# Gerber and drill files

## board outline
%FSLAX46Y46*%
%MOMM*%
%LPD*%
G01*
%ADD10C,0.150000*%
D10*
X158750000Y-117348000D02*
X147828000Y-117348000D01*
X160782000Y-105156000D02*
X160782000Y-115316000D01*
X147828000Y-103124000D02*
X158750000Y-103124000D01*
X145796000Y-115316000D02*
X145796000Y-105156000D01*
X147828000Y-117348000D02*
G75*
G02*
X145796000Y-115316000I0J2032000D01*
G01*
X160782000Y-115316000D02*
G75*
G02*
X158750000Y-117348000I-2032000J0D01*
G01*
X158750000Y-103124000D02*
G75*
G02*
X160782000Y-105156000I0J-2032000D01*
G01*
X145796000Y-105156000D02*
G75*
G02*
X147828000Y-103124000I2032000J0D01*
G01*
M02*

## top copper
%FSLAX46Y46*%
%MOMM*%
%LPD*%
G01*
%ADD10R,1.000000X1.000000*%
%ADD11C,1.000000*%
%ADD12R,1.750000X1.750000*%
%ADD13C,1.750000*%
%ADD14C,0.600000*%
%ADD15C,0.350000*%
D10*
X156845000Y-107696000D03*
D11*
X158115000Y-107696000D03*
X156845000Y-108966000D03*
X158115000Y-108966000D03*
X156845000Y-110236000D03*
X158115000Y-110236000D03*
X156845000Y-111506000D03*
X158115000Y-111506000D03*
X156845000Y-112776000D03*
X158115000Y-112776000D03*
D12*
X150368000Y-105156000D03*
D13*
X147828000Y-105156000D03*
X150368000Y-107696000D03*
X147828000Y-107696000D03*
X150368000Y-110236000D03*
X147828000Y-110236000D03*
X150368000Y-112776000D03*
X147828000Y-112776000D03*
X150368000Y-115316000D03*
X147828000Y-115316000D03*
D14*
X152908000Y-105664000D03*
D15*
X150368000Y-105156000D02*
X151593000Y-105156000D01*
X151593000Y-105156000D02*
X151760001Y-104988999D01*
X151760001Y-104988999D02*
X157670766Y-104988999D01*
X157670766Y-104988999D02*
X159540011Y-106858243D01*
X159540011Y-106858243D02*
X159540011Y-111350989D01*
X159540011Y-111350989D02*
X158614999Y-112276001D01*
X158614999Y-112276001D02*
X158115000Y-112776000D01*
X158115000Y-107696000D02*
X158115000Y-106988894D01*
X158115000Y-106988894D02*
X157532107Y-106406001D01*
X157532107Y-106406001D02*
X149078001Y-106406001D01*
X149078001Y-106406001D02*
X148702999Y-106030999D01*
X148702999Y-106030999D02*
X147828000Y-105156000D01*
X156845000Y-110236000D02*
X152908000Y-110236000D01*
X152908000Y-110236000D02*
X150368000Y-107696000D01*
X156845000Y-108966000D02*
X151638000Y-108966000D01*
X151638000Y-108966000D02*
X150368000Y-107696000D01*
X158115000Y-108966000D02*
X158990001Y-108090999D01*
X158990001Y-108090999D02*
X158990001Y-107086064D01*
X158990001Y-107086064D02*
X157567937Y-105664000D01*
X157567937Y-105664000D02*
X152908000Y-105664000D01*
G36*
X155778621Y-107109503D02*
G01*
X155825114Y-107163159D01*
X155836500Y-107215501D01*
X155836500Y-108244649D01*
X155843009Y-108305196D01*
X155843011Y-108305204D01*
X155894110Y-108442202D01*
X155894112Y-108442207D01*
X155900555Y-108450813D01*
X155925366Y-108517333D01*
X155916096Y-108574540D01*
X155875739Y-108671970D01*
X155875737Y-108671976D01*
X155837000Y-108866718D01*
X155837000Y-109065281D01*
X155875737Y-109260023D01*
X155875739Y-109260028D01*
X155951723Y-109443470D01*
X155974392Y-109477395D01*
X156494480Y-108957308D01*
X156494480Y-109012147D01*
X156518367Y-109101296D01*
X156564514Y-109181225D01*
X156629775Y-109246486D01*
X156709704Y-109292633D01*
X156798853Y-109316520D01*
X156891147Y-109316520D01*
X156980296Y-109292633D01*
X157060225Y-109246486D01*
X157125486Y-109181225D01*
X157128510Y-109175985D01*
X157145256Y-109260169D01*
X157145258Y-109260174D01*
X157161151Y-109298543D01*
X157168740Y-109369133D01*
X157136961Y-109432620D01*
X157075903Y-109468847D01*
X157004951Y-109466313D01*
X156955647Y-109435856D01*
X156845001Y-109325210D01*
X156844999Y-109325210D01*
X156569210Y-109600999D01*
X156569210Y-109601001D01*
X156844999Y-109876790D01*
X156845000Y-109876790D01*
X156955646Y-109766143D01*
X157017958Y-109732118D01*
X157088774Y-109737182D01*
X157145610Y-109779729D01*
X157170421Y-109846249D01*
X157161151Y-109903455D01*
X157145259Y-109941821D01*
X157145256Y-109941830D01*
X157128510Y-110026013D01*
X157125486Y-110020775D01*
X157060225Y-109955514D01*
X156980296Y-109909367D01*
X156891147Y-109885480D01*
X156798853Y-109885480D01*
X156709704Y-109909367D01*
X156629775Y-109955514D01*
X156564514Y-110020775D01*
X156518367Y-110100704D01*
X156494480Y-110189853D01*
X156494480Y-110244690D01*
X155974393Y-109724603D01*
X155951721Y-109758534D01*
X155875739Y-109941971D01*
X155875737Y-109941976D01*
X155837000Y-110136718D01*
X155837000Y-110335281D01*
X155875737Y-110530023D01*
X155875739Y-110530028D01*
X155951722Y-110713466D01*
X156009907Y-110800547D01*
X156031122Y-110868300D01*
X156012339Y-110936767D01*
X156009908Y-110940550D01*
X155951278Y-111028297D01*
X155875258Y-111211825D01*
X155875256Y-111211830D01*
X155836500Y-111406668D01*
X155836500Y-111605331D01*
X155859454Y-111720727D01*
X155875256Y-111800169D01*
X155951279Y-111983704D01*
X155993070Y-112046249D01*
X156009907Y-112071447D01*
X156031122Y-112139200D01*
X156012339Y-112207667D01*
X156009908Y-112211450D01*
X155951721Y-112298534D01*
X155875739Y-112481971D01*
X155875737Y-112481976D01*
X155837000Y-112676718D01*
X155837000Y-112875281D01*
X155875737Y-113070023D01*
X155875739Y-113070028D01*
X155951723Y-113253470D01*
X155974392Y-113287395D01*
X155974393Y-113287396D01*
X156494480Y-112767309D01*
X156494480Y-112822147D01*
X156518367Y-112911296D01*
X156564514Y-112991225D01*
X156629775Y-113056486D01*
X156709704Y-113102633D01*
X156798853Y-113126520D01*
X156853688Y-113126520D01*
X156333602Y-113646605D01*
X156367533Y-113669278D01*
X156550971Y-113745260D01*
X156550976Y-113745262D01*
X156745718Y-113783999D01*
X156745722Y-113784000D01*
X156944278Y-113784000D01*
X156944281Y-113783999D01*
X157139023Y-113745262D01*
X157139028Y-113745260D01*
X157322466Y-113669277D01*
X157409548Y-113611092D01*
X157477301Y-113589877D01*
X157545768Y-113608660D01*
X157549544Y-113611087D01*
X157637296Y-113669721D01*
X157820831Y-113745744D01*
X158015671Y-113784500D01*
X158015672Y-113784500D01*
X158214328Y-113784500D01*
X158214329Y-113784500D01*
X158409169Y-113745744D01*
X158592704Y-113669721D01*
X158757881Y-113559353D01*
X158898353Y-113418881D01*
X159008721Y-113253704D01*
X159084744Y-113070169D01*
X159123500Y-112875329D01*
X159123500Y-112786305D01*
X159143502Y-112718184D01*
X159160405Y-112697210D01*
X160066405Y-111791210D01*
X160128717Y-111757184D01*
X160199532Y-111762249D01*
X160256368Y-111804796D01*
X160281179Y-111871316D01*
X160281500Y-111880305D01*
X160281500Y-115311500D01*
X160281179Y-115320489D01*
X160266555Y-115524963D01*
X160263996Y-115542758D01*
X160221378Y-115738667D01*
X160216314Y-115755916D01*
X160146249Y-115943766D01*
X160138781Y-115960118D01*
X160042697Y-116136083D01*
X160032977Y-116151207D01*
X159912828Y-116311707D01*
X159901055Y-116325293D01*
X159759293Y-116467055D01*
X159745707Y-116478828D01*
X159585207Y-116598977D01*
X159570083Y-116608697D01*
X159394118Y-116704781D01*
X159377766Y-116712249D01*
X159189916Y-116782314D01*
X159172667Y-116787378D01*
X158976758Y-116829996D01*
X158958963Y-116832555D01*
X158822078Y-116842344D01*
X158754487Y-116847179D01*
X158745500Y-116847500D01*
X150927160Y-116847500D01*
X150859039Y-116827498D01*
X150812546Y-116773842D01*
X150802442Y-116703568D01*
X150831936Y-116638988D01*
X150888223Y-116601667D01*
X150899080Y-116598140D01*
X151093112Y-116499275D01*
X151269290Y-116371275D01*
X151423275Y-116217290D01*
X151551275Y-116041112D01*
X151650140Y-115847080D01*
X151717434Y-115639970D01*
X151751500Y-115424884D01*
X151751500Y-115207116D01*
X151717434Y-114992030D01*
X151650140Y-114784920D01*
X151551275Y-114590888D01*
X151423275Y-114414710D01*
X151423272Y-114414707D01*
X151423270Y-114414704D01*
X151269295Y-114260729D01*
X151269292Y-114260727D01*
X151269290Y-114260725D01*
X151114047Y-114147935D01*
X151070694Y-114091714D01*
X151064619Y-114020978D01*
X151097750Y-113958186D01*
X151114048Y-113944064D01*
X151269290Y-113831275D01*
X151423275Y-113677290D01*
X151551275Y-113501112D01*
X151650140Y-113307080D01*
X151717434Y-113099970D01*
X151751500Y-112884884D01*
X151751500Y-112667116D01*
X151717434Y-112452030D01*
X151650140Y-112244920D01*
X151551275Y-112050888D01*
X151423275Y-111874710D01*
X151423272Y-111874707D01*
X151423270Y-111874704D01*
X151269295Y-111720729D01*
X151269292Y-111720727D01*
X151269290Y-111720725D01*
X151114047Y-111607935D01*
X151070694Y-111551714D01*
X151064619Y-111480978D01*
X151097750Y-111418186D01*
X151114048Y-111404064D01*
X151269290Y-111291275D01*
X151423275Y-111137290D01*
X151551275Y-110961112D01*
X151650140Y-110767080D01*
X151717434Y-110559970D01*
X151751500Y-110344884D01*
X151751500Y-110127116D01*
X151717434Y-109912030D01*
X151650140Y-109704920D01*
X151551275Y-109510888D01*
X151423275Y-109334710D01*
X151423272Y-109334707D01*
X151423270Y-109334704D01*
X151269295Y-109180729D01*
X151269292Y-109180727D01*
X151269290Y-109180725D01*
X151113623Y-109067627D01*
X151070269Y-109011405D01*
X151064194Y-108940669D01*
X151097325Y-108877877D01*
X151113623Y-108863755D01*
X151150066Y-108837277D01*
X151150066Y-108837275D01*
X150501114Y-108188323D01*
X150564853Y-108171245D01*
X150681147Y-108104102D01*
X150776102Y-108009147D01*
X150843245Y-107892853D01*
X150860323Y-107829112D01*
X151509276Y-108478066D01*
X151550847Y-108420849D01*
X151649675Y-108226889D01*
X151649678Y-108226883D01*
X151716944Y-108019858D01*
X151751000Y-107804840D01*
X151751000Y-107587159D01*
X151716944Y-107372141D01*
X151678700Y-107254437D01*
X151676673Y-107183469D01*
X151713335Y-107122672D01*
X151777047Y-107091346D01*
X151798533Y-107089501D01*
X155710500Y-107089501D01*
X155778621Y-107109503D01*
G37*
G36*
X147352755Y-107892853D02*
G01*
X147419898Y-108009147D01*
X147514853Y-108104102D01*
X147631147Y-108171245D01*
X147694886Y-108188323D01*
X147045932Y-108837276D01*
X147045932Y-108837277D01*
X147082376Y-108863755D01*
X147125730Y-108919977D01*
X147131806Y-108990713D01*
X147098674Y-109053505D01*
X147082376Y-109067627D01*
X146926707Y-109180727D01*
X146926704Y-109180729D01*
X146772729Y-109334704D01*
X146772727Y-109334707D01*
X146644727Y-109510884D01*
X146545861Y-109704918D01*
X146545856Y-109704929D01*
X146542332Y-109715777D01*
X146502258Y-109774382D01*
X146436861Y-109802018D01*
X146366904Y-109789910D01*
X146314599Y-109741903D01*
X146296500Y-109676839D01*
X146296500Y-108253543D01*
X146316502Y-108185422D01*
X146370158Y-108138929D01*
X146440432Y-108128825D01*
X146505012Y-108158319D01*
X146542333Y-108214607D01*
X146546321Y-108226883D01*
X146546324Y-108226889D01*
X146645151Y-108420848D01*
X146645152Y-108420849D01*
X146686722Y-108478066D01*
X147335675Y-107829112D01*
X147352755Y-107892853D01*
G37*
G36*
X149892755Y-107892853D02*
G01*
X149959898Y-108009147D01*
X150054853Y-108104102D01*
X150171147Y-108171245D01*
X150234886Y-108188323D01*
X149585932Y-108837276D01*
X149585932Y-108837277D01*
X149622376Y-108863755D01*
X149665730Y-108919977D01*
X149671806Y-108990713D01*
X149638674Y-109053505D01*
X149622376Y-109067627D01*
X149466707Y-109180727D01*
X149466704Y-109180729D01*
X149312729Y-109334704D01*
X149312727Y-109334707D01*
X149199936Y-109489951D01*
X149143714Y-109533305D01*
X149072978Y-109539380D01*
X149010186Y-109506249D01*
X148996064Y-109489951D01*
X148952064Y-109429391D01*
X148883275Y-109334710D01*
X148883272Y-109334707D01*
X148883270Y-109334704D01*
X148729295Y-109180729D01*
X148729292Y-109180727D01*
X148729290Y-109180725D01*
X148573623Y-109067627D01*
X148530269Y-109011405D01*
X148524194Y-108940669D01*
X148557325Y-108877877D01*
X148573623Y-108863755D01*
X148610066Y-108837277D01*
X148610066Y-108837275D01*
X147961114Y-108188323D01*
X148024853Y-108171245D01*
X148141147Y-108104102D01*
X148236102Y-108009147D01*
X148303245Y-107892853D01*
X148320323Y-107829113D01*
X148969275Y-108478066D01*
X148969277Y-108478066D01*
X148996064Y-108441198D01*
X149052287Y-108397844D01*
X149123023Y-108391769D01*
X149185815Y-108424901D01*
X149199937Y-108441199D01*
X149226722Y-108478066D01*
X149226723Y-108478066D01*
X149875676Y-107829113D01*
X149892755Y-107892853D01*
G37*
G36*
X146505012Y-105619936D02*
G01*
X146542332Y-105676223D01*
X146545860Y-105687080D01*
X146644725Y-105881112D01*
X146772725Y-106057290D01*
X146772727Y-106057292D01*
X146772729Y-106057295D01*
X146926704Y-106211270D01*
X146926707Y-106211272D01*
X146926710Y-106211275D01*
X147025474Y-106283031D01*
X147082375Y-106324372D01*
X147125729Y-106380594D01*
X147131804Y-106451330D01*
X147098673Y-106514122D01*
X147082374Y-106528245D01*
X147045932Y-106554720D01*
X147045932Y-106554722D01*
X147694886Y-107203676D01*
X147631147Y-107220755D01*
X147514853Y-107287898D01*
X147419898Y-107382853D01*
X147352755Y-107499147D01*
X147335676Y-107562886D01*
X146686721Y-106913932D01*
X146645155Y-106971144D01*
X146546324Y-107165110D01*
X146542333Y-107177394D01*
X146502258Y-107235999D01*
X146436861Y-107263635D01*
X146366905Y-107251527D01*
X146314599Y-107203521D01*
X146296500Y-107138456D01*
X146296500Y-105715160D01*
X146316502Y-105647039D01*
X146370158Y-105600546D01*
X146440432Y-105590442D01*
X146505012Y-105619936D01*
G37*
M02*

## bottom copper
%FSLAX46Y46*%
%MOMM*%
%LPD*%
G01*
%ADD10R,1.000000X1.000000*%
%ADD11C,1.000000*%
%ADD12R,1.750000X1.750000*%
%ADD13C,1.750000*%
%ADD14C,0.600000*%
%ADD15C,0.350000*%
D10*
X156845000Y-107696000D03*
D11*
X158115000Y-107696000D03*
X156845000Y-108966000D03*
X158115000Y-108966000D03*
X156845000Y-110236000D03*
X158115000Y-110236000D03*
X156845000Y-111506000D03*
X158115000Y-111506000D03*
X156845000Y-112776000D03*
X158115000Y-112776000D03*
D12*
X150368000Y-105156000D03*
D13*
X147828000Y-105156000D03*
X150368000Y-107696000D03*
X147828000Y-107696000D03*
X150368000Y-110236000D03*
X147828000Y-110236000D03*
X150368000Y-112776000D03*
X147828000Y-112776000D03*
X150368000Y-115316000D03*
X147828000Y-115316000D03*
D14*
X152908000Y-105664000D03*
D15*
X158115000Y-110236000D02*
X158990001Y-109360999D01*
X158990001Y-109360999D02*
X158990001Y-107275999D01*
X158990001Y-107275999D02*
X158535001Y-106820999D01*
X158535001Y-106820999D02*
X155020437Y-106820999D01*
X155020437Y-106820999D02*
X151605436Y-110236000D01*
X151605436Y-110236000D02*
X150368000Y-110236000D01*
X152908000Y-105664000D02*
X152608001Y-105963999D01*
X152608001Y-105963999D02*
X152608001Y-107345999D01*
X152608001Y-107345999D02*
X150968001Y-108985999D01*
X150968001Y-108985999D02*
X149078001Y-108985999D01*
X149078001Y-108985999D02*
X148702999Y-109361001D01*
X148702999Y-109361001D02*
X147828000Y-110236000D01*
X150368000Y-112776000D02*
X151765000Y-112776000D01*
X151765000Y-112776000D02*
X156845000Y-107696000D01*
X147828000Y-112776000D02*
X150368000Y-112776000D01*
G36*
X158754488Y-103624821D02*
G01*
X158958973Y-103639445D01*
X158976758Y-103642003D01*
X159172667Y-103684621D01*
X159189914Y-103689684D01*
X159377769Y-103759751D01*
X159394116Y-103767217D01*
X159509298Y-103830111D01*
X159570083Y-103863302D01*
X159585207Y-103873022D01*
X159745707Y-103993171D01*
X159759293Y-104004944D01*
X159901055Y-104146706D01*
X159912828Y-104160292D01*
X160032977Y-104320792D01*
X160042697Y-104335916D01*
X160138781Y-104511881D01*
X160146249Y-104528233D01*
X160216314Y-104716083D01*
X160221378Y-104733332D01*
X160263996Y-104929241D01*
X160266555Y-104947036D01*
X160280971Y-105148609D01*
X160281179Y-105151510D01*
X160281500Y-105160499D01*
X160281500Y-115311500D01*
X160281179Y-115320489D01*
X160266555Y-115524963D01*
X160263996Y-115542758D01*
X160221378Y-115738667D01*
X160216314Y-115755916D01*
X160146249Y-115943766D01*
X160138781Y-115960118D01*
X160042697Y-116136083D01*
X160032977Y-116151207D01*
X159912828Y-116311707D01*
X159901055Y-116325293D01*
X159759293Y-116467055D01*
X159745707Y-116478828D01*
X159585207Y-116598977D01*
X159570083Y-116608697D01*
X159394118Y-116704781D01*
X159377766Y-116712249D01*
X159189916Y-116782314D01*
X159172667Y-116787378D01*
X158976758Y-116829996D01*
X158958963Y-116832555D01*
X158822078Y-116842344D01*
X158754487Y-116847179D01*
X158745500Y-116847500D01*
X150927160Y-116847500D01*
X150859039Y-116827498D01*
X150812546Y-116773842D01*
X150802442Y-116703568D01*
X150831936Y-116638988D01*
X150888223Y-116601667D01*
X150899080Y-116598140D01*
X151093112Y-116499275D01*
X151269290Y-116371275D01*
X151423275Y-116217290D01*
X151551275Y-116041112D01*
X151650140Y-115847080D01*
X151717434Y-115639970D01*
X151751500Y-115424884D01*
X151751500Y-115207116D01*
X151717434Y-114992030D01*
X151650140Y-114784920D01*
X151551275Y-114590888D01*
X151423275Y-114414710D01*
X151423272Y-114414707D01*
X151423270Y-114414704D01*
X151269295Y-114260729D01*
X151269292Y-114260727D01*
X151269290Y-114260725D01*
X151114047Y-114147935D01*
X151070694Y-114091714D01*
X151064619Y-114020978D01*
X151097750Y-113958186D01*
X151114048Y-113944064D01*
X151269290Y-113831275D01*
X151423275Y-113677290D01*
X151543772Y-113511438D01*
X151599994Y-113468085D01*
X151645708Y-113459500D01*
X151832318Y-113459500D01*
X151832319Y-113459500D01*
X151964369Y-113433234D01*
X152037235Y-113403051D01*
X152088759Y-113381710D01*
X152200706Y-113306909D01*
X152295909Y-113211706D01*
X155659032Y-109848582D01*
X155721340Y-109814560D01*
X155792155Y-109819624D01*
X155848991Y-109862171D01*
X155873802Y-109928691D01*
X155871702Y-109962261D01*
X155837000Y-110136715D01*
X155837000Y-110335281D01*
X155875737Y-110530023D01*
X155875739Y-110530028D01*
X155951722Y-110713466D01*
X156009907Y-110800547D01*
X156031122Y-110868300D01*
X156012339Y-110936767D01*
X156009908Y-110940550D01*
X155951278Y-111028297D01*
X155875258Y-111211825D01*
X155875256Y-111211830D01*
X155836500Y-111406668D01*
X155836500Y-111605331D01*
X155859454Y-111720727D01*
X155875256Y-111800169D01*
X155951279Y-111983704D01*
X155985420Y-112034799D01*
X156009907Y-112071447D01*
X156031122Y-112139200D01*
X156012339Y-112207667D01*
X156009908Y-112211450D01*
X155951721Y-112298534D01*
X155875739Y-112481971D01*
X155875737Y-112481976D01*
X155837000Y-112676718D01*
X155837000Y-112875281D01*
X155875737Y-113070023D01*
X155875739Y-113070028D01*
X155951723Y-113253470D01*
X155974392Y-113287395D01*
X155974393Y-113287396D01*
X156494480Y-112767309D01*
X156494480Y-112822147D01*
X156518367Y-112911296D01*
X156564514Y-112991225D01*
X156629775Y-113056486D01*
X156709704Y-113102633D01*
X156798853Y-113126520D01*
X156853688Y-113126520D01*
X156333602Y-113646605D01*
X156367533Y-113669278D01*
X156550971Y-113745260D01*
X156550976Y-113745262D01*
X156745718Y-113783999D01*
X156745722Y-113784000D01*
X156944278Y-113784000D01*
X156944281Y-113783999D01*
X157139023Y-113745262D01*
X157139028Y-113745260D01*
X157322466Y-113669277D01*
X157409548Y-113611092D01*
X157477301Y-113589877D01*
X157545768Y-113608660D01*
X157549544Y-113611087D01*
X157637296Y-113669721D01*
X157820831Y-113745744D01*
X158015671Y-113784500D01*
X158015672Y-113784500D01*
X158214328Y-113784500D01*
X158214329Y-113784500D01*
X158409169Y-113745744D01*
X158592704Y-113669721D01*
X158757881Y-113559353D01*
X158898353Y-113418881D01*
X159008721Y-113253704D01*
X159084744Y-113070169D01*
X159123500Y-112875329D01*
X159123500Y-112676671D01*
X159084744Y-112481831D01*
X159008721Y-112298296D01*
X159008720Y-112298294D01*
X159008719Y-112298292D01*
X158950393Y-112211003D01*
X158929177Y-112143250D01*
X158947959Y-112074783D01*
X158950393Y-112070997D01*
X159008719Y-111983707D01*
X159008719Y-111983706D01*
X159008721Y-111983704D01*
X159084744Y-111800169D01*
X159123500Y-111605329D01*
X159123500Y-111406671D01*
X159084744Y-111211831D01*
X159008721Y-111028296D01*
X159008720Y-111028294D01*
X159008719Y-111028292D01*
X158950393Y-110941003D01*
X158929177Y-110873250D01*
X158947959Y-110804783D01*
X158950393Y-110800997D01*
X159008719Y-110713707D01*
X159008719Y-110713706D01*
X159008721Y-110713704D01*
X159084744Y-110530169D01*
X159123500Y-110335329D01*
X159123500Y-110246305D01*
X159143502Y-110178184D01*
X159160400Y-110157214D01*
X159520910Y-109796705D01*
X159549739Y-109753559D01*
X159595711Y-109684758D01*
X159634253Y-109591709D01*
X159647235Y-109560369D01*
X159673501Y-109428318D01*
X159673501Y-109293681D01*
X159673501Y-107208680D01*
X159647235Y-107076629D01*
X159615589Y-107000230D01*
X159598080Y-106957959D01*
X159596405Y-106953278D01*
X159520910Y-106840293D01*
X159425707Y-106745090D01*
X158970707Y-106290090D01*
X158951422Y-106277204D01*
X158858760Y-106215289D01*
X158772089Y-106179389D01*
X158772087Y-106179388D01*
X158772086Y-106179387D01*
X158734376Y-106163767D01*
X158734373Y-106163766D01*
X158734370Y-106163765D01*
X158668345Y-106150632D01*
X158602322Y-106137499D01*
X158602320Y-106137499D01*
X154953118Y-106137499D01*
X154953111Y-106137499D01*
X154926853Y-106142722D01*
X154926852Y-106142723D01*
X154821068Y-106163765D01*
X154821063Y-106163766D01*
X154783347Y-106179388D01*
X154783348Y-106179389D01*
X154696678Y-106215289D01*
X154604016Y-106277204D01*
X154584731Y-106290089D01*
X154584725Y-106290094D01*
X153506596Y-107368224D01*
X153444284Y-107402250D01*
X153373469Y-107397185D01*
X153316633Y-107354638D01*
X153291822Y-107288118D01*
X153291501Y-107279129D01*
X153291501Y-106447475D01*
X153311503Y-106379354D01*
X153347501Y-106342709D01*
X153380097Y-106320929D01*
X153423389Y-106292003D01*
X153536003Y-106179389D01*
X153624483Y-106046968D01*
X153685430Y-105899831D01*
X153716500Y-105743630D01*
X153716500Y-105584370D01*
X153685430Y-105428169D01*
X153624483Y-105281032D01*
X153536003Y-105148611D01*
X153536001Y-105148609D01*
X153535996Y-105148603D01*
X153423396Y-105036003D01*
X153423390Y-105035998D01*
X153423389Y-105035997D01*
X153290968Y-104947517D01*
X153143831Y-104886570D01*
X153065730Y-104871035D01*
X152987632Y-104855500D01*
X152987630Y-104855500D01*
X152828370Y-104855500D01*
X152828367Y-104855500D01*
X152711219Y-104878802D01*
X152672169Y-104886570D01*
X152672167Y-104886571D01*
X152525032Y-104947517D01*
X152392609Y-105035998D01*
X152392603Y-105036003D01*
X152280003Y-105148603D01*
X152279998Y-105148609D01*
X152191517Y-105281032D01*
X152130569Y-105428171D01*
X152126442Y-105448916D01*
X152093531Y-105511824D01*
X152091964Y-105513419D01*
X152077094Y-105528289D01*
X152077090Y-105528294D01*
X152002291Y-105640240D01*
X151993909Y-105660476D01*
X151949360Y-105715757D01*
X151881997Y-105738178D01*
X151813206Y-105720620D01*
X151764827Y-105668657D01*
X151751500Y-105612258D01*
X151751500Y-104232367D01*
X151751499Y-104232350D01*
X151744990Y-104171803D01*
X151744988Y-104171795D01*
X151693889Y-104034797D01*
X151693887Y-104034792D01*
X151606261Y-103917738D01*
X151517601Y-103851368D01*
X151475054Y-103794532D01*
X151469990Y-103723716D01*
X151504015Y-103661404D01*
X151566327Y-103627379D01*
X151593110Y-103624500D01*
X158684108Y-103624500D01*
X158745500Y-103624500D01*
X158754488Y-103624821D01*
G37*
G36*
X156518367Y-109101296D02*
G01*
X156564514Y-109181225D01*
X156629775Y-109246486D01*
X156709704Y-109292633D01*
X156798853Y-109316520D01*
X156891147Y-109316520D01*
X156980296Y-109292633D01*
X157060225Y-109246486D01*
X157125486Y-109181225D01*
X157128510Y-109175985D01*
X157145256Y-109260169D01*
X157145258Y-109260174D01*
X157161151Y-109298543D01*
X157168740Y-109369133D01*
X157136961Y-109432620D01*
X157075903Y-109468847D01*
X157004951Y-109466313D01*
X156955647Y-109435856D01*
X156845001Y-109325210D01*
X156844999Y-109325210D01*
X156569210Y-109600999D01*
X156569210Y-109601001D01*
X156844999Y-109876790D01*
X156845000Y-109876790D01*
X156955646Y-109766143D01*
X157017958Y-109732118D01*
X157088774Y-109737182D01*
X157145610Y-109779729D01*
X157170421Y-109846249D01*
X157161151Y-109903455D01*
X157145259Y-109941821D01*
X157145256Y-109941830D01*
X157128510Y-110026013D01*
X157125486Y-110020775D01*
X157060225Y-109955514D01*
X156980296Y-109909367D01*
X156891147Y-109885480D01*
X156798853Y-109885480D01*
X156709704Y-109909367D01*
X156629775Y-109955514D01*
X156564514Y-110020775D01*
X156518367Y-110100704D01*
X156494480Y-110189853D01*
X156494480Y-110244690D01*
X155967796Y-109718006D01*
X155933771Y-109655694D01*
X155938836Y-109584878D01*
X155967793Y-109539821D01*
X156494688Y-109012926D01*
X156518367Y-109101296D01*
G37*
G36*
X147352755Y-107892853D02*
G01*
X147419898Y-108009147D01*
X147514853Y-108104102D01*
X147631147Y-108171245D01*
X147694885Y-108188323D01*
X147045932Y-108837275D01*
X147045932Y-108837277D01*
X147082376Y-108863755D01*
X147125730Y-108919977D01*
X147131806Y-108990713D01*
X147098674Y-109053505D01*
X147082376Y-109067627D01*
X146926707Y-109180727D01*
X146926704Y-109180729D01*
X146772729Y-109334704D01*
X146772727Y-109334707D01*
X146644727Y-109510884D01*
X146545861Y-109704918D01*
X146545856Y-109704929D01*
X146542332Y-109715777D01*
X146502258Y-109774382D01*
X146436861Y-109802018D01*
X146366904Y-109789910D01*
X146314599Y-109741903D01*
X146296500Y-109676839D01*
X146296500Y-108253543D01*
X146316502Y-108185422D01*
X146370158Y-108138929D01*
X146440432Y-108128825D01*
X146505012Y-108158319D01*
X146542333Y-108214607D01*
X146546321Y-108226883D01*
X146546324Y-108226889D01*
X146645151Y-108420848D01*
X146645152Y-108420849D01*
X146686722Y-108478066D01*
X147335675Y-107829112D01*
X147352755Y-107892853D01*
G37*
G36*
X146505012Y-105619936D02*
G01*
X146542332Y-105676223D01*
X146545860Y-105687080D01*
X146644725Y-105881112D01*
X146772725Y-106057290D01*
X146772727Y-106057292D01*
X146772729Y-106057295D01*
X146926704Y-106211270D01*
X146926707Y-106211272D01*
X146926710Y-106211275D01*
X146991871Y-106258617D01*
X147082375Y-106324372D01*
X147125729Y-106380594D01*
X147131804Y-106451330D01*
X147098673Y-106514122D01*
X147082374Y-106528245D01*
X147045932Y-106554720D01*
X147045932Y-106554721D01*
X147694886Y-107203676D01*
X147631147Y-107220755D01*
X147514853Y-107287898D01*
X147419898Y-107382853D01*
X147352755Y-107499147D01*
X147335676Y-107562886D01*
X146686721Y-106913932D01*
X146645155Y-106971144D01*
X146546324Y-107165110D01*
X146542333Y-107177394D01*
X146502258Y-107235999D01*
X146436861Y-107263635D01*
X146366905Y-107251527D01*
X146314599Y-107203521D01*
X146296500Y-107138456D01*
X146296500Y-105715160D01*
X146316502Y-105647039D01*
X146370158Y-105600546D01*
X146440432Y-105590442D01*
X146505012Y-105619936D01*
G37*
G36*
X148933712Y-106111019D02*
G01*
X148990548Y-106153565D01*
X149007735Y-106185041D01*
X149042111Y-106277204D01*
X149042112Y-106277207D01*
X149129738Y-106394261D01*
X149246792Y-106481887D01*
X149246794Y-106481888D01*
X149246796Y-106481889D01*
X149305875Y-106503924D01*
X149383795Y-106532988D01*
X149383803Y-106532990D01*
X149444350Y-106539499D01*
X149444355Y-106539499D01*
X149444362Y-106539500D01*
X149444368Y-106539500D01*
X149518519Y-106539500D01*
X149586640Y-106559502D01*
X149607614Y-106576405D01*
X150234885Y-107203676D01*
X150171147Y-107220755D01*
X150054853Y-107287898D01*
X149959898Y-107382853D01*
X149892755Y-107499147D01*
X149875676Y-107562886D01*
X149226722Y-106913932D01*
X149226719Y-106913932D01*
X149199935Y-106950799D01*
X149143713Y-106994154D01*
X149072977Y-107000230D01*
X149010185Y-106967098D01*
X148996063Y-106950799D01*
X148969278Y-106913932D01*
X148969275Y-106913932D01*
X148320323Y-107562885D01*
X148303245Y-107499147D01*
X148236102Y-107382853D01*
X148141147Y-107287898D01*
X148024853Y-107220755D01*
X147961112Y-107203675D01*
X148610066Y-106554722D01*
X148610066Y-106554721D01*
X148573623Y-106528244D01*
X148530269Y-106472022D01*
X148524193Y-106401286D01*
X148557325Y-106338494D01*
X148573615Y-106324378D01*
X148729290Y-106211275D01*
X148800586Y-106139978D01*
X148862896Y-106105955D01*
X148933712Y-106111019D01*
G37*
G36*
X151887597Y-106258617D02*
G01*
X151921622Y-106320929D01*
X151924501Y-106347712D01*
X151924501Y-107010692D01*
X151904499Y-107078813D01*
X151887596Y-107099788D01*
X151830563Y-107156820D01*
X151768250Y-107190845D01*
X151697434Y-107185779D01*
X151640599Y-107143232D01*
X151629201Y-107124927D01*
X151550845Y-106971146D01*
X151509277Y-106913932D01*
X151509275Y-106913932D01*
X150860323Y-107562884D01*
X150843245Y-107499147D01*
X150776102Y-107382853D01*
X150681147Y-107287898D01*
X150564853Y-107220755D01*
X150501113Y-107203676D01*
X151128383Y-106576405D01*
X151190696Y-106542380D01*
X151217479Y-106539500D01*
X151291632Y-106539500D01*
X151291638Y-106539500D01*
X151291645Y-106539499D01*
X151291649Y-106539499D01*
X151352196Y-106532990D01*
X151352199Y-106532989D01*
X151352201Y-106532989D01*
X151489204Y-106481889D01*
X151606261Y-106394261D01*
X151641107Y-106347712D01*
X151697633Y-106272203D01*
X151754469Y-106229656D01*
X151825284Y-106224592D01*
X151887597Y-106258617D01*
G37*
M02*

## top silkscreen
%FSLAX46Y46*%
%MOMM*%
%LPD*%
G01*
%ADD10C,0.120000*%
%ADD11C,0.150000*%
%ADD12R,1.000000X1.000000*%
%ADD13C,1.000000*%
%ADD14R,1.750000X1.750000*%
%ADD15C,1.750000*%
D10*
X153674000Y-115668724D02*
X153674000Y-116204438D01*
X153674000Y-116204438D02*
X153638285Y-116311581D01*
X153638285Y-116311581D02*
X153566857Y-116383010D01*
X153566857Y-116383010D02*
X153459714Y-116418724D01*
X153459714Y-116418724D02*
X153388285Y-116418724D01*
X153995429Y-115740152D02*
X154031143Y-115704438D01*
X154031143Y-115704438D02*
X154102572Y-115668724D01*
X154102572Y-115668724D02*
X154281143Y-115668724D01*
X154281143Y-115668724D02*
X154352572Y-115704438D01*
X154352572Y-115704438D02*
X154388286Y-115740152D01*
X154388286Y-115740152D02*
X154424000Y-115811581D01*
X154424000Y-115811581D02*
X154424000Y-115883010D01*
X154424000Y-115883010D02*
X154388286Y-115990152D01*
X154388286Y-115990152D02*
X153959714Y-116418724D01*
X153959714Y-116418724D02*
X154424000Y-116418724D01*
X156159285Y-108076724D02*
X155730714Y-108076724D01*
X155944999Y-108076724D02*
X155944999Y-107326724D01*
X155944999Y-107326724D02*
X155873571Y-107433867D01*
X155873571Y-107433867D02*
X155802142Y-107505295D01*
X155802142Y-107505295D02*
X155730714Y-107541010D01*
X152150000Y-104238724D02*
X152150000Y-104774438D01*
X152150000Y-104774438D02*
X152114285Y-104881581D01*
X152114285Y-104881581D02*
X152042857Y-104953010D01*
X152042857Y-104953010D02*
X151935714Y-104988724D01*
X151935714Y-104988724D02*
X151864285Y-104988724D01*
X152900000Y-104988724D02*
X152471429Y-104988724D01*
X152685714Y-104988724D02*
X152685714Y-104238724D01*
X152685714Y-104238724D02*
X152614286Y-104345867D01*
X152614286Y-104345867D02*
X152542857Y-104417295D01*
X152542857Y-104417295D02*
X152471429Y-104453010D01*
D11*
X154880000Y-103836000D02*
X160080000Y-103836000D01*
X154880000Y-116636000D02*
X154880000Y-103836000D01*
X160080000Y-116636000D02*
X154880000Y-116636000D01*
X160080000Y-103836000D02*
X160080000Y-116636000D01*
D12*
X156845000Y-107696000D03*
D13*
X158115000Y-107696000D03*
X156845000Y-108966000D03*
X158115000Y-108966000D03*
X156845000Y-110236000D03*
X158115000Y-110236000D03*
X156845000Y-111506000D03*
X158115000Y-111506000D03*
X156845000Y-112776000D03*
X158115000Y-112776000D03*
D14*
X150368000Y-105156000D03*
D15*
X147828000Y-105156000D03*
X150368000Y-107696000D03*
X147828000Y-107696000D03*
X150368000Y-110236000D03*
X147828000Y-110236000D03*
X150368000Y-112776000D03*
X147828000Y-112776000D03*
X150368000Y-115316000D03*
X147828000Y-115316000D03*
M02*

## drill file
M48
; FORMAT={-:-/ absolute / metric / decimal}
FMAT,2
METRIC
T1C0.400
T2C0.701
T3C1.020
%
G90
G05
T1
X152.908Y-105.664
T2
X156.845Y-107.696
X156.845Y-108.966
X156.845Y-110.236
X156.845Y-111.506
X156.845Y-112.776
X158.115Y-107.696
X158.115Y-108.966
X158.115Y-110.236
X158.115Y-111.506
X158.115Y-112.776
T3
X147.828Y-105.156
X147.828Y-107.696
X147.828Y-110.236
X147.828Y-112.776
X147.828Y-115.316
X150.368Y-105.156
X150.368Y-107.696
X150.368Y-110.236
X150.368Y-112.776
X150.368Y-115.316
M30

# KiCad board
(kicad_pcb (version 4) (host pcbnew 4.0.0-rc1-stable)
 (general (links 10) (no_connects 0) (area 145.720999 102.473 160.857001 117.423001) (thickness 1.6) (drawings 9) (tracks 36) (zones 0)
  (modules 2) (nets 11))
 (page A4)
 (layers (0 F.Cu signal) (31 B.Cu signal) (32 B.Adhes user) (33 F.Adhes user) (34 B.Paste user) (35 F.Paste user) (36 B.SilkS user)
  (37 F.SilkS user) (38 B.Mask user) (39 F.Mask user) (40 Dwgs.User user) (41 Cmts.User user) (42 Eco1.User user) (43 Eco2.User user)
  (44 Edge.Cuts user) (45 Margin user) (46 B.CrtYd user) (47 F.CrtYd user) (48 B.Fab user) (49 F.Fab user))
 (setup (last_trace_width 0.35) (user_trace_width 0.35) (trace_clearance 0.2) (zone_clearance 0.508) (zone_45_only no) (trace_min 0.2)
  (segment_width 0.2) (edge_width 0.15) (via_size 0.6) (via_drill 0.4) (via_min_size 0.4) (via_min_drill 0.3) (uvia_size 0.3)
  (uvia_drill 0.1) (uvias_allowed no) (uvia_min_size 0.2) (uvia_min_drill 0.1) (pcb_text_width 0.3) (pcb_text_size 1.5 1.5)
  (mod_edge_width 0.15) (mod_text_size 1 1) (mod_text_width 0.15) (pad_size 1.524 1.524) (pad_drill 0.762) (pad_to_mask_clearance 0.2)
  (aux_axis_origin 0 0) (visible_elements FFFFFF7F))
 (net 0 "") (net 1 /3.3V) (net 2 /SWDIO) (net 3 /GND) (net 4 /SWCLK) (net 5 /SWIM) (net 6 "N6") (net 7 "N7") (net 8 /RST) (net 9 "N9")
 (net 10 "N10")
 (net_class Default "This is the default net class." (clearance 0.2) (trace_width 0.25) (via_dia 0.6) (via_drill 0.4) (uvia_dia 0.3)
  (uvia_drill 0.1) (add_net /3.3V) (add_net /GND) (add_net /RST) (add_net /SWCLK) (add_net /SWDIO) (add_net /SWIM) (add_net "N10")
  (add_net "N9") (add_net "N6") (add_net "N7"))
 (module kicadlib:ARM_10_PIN (layer F.Cu) (at 157.48 110.236)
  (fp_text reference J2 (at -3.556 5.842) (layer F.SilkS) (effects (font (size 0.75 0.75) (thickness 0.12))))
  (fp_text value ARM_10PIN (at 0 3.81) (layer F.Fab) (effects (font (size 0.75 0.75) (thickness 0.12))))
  (fp_line (start -2.6 -6.4) (end 2.6 -6.4) (layer F.SilkS) (width 0.15))
  (fp_line (start -2.6 6.4) (end -2.6 -6.4) (layer F.SilkS) (width 0.15))
  (fp_line (start 2.6 6.4) (end -2.6 6.4) (layer F.SilkS) (width 0.15))
  (fp_line (start 2.6 -6.4) (end 2.6 6.4) (layer F.SilkS) (width 0.15))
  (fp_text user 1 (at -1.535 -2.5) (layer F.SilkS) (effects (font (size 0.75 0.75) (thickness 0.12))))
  (pad 1 thru_hole rect (at -0.635 -2.54) (size 1 1) (drill 0.70104) (layers *.Cu *.Mask F.SilkS) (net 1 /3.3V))
  (pad 2 thru_hole circle (at 0.635 -2.54) (size 1 1) (drill 0.70104) (layers *.Cu *.Mask F.SilkS) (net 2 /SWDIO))
  (pad 3 thru_hole circle (at -0.635 -1.27) (size 1 1) (drill 0.70104) (layers *.Cu *.Mask F.SilkS) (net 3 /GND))
  (pad 4 thru_hole circle (at 0.635 -1.27) (size 1 1) (drill 0.70104) (layers *.Cu *.Mask F.SilkS) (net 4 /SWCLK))
  (pad 5 thru_hole circle (at -0.635 0) (size 1 1) (drill 0.70104) (layers *.Cu *.Mask F.SilkS) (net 3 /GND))
  (pad 6 thru_hole circle (at 0.635 0) (size 1 1) (drill 0.70104) (layers *.Cu *.Mask F.SilkS) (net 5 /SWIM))
  (pad 7 thru_hole circle (at -0.635 1.27) (size 1 1) (drill 0.70104) (layers *.Cu *.Mask F.SilkS) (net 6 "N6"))
  (pad 8 thru_hole circle (at 0.635 1.27) (size 1 1) (drill 0.70104) (layers *.Cu *.Mask F.SilkS) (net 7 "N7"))
  (pad 9 thru_hole circle (at -0.635 2.54) (size 1 1) (drill 0.70104) (layers *.Cu *.Mask F.SilkS) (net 3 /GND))
  (pad 10 thru_hole circle (at 0.635 2.54) (size 1 1) (drill 0.70104) (layers *.Cu *.Mask F.SilkS) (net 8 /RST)))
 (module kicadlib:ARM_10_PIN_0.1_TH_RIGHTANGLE (layer F.Cu) (at 150.368 105.156)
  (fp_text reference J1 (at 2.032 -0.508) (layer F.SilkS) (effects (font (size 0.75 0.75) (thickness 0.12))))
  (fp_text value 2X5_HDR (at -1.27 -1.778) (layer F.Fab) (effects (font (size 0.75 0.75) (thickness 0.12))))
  (pad 1 thru_hole rect (at 0 0) (size 1.75 1.75) (drill 1.02) (layers *.Cu *.Mask F.SilkS) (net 8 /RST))
  (pad 2 thru_hole circle (at -2.54 0) (size 1.75 1.75) (drill 1.02) (layers *.Cu *.Mask F.SilkS) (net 2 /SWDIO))
  (pad 3 thru_hole circle (at 0 2.54) (size 1.75 1.75) (drill 1.02) (layers *.Cu *.Mask F.SilkS) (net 3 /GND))
  (pad 4 thru_hole circle (at -2.54 2.54) (size 1.75 1.75) (drill 1.02) (layers *.Cu *.Mask F.SilkS) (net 3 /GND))
  (pad 5 thru_hole circle (at 0 5.08) (size 1.75 1.75) (drill 1.02) (layers *.Cu *.Mask F.SilkS) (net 5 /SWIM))
  (pad 6 thru_hole circle (at -2.54 5.08) (size 1.75 1.75) (drill 1.02) (layers *.Cu *.Mask F.SilkS) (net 4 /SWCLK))
  (pad 7 thru_hole circle (at 0 7.62) (size 1.75 1.75) (drill 1.02) (layers *.Cu *.Mask F.SilkS) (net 1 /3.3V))
  (pad 8 thru_hole circle (at -2.54 7.62) (size 1.75 1.75) (drill 1.02) (layers *.Cu *.Mask F.SilkS) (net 1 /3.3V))
  (pad 9 thru_hole circle (at 0 10.16) (size 1.75 1.75) (drill 1.02) (layers *.Cu *.Mask F.SilkS) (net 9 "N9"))
  (pad 10 thru_hole circle (at -2.54 10.16) (size 1.75 1.75) (drill 1.02) (layers *.Cu *.Mask F.SilkS) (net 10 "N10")))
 (gr_line (start 158.75 117.348) (end 147.828 117.348) (angle 90) (layer Edge.Cuts) (width 0.15))
 (gr_line (start 160.782 105.156) (end 160.782 115.316) (angle 90) (layer Edge.Cuts) (width 0.15))
 (gr_line (start 147.828 103.124) (end 158.75 103.124) (angle 90) (layer Edge.Cuts) (width 0.15))
 (gr_line (start 145.796 115.316) (end 145.796 105.156) (angle 90) (layer Edge.Cuts) (width 0.15))
 (gr_arc (start 147.828 115.316) (end 147.828 117.348) (angle 90) (layer Edge.Cuts) (width 0.15))
 (gr_arc (start 158.75 115.316) (end 160.782 115.316) (angle 90) (layer Edge.Cuts) (width 0.15))
 (gr_arc (start 158.75 105.156) (end 158.75 103.124) (angle 90) (layer Edge.Cuts) (width 0.15))
 (gr_arc (start 147.828 105.156) (end 145.796 105.156) (angle 90) (layer Edge.Cuts) (width 0.15))
 (segment (start 150.368 105.156) (end 151.593 105.156) (width 0.35) (layer F.Cu) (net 8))
 (segment (start 151.593 105.156) (end 151.760001 104.988999) (width 0.35) (layer F.Cu) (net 8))
 (segment (start 151.760001 104.988999) (end 157.670766 104.988999) (width 0.35) (layer F.Cu) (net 8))
 (segment (start 157.670766 104.988999) (end 159.540011 106.858243) (width 0.35) (layer F.Cu) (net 8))
 (segment (start 159.540011 106.858243) (end 159.540011 111.350989) (width 0.35) (layer F.Cu) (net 8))
 (segment (start 159.540011 111.350989) (end 158.614999 112.276001) (width 0.35) (layer F.Cu) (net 8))
 (segment (start 158.614999 112.276001) (end 158.115 112.776) (width 0.35) (layer F.Cu) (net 8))
 (segment (start 158.115 107.696) (end 158.115 106.988894) (width 0.35) (layer F.Cu) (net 2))
 (segment (start 158.115 106.988894) (end 157.532107 106.406001) (width 0.35) (layer F.Cu) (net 2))
 (segment (start 157.532107 106.406001) (end 149.078001 106.406001) (width 0.35) (layer F.Cu) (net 2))
 (segment (start 149.078001 106.406001) (end 148.702999 106.030999) (width 0.35) (layer F.Cu) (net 2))
 (segment (start 148.702999 106.030999) (end 147.828 105.156) (width 0.35) (layer F.Cu) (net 2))
 (segment (start 156.845 110.236) (end 152.908 110.236) (width 0.35) (layer F.Cu) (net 3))
 (segment (start 152.908 110.236) (end 150.368 107.696) (width 0.35) (layer F.Cu) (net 3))
 (segment (start 156.845 108.966) (end 151.638 108.966) (width 0.35) (layer F.Cu) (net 3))
 (segment (start 151.638 108.966) (end 150.368 107.696) (width 0.35) (layer F.Cu) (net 3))
 (segment (start 158.115 110.236) (end 158.990001 109.360999) (width 0.35) (layer B.Cu) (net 5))
 (segment (start 158.990001 109.360999) (end 158.990001 107.275999) (width 0.35) (layer B.Cu) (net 5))
 (segment (start 158.990001 107.275999) (end 158.535001 106.820999) (width 0.35) (layer B.Cu) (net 5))
 (segment (start 158.535001 106.820999) (end 155.020437 106.820999) (width 0.35) (layer B.Cu) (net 5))
 (segment (start 155.020437 106.820999) (end 151.605436 110.236) (width 0.35) (layer B.Cu) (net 5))
 (segment (start 151.605436 110.236) (end 150.368 110.236) (width 0.35) (layer B.Cu) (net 5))
 (segment (start 152.908 105.664) (end 152.608001 105.963999) (width 0.35) (layer B.Cu) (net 4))
 (segment (start 152.608001 105.963999) (end 152.608001 107.345999) (width 0.35) (layer B.Cu) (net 4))
 (segment (start 152.608001 107.345999) (end 150.968001 108.985999) (width 0.35) (layer B.Cu) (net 4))
 (segment (start 150.968001 108.985999) (end 149.078001 108.985999) (width 0.35) (layer B.Cu) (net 4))
 (segment (start 149.078001 108.985999) (end 148.702999 109.361001) (width 0.35) (layer B.Cu) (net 4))
 (segment (start 148.702999 109.361001) (end 147.828 110.236) (width 0.35) (layer B.Cu) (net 4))
 (segment (start 158.115 108.966) (end 158.990001 108.090999) (width 0.35) (layer F.Cu) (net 4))
 (segment (start 158.990001 108.090999) (end 158.990001 107.086064) (width 0.35) (layer F.Cu) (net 4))
 (segment (start 158.990001 107.086064) (end 157.567937 105.664) (width 0.35) (layer F.Cu) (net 4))
 (segment (start 157.567937 105.664) (end 152.908 105.664) (width 0.35) (layer F.Cu) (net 4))
 (via (at 152.908 105.664) (size 0.6) (drill 0.4) (layers F.Cu B.Cu) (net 4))
 (segment (start 150.368 112.776) (end 151.765 112.776) (width 0.35) (layer B.Cu) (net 1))
 (segment (start 151.765 112.776) (end 156.845 107.696) (width 0.35) (layer B.Cu) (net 1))
 (segment (start 147.828 112.776) (end 150.368 112.776) (width 0.35) (layer B.Cu) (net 1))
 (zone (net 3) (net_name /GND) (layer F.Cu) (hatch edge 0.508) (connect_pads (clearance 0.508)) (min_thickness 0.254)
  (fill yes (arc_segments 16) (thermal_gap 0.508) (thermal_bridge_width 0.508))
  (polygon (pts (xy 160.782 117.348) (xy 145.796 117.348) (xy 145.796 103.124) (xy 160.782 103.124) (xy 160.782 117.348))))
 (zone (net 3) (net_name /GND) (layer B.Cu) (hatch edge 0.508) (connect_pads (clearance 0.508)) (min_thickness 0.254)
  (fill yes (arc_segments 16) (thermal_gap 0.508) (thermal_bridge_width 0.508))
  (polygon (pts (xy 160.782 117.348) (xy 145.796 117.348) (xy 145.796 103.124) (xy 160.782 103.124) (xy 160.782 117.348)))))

